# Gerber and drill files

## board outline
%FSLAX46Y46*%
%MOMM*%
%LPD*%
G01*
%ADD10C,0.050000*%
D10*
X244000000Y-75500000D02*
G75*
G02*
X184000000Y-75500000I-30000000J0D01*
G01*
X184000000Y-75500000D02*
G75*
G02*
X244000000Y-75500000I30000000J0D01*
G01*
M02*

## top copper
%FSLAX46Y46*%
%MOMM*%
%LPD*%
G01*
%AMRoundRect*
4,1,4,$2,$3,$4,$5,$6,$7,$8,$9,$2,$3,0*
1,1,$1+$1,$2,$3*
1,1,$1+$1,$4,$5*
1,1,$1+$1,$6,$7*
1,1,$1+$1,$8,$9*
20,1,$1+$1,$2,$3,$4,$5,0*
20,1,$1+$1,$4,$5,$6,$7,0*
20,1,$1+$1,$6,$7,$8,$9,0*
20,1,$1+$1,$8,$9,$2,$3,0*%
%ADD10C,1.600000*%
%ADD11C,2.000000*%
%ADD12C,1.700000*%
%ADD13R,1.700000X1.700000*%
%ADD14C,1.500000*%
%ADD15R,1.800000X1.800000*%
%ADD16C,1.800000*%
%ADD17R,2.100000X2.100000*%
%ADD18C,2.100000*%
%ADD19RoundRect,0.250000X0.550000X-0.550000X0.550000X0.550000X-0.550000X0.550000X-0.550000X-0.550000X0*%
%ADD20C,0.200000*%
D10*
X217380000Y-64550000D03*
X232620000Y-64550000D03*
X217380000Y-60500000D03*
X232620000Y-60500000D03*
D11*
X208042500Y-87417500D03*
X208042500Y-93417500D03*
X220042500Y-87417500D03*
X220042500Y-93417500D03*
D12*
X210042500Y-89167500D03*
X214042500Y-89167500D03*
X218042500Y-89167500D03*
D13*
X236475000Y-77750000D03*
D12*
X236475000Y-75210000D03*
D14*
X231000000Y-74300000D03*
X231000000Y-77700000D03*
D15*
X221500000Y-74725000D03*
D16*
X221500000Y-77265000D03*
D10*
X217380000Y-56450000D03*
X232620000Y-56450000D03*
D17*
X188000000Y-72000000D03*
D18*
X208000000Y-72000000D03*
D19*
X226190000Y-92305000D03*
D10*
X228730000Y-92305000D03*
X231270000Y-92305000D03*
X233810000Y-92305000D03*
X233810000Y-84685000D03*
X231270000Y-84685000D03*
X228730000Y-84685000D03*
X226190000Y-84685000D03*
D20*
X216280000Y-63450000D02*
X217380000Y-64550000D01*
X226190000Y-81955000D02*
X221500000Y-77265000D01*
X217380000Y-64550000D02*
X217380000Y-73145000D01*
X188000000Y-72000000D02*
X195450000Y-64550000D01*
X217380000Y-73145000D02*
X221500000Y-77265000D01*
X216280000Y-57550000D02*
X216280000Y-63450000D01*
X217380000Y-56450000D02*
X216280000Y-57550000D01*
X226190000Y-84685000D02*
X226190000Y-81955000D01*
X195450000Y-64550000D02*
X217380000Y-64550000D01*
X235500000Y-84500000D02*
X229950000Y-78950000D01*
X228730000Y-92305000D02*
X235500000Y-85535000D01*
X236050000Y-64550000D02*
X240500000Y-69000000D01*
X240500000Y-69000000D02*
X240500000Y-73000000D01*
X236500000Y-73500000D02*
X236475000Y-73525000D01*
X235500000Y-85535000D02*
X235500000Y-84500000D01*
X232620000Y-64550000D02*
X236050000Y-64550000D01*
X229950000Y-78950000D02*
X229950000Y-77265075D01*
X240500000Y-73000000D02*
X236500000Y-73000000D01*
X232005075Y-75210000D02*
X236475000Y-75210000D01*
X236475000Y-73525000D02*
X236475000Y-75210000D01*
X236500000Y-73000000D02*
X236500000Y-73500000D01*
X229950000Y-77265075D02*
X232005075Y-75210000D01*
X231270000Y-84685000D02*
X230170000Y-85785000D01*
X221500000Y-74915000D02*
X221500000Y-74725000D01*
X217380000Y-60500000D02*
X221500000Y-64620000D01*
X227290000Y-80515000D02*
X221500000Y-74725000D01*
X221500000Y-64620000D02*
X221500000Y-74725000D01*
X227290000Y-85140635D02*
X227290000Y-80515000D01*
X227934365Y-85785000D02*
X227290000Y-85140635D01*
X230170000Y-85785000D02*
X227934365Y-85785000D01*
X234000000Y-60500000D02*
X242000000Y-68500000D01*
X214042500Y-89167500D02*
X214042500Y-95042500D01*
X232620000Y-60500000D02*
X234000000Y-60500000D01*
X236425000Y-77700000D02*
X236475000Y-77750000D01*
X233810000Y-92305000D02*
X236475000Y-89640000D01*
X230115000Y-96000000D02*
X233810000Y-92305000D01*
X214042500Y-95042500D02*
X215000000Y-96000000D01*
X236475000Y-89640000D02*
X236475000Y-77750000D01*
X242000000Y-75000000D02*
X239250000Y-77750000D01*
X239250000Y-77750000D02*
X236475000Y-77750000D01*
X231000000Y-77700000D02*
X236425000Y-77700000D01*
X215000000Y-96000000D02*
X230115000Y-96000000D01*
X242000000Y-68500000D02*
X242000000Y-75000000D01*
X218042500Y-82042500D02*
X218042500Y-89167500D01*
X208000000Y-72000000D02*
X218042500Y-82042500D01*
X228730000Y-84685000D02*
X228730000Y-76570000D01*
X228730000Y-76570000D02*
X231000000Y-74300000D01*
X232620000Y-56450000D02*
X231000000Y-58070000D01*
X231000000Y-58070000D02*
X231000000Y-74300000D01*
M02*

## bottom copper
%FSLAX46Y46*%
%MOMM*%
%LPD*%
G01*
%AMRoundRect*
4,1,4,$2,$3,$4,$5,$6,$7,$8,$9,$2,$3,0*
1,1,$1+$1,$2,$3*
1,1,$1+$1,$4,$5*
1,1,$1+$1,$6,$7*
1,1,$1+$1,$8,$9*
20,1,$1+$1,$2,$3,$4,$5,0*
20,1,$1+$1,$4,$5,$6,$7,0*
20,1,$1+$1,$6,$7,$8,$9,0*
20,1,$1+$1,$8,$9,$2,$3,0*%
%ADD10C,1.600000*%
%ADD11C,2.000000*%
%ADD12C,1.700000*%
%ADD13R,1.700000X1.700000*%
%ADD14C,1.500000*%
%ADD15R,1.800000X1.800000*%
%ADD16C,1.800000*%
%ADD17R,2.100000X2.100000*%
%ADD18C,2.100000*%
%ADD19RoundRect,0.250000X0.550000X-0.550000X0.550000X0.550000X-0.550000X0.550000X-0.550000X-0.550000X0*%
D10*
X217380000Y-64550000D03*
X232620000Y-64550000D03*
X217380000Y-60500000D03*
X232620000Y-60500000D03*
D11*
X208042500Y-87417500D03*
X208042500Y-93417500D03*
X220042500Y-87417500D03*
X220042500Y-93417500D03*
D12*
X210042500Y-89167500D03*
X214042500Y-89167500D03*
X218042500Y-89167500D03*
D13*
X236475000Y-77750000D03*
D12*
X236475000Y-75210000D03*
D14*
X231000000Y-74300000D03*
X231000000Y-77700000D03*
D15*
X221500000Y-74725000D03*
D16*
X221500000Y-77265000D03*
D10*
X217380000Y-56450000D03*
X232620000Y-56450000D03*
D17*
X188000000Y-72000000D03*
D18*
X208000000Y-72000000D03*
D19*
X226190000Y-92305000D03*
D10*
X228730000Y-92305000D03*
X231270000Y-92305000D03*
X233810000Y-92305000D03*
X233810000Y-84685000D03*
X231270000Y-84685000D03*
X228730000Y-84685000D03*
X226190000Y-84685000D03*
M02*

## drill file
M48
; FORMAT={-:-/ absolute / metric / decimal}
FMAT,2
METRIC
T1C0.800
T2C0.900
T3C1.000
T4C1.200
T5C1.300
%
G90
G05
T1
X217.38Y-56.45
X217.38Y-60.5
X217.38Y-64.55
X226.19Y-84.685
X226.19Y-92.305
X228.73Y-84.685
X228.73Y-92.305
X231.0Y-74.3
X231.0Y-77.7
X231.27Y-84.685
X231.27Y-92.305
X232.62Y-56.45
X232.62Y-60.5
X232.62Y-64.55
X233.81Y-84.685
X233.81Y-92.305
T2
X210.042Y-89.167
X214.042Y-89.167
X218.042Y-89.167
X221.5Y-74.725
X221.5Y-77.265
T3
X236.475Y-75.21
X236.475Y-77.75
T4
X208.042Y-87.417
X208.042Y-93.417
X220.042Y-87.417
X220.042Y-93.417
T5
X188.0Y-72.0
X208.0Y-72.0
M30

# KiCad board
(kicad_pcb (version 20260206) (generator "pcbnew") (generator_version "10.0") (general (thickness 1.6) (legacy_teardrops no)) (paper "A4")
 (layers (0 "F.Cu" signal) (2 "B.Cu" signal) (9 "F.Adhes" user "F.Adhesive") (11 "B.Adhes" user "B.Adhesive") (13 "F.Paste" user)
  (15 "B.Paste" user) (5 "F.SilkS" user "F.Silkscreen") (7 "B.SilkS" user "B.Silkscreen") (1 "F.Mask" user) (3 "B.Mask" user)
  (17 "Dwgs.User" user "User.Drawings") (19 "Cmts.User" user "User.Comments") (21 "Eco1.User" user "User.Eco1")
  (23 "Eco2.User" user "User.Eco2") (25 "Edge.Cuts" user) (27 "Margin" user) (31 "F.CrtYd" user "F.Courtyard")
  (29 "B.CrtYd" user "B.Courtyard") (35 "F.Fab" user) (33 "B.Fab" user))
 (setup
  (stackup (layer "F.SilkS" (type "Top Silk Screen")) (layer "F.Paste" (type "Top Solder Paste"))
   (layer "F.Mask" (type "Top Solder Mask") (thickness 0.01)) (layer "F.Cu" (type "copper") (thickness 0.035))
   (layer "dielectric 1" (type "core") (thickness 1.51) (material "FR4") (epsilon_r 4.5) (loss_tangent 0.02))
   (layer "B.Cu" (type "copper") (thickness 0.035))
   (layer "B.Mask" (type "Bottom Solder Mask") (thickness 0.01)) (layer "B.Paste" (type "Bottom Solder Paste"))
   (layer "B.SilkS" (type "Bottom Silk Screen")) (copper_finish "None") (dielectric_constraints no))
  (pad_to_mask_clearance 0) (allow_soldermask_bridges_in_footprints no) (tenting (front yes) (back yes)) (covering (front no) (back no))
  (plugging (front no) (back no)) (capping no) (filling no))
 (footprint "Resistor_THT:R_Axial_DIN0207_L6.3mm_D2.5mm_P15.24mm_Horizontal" (layer "F.Cu") (at 217.38 64.55)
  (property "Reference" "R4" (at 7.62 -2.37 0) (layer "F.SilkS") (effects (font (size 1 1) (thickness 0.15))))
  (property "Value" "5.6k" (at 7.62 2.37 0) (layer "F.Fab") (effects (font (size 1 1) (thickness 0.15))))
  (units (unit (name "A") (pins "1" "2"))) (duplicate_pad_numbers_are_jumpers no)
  (pad "1" thru_hole circle (at 0 0) (size 1.6 1.6) (drill 0.8) (layers "*.Cu" "*.Mask") (remove_unused_layers no) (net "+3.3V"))
  (pad "2" thru_hole circle (at 15.24 0) (size 1.6 1.6) (drill 0.8) (layers "*.Cu" "*.Mask") (remove_unused_layers no) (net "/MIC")))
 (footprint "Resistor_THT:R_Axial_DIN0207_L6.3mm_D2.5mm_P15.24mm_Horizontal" (layer "F.Cu") (at 217.38 60.5)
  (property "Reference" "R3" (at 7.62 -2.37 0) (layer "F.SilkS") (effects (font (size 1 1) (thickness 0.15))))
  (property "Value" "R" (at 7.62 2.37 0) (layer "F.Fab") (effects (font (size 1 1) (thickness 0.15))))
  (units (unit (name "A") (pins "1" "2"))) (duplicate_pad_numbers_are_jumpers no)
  (pad "1" thru_hole circle (at 0 0) (size 1.6 1.6) (drill 0.8) (layers "*.Cu" "*.Mask") (remove_unused_layers no) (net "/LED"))
  (pad "2" thru_hole circle (at 15.24 0) (size 1.6 1.6) (drill 0.8) (layers "*.Cu" "*.Mask") (remove_unused_layers no) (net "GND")))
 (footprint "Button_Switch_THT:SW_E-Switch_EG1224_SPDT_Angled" (layer "F.Cu") (at 210.0425 89.1675)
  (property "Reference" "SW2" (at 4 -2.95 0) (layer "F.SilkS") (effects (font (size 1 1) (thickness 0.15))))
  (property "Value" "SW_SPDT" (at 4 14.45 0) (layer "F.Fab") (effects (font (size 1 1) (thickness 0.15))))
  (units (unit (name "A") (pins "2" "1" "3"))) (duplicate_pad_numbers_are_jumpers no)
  (pad "" thru_hole circle (at -2 -1.75) (size 2 2) (drill 1.2) (layers "*.Cu" "*.Mask") (remove_unused_layers no))
  (pad "" thru_hole circle (at -2 4.25) (size 2 2) (drill 1.2) (layers "*.Cu" "*.Mask") (remove_unused_layers no))
  (pad "" thru_hole circle (at 10 -1.75) (size 2 2) (drill 1.2) (layers "*.Cu" "*.Mask") (remove_unused_layers no))
  (pad "" thru_hole circle (at 10 4.25) (size 2 2) (drill 1.2) (layers "*.Cu" "*.Mask") (remove_unused_layers no))
  (pad "1" thru_hole circle (at 0 0) (size 1.7 1.7) (drill 0.9) (layers "*.Cu" "*.Mask") (remove_unused_layers no)
   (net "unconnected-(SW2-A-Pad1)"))
  (pad "2" thru_hole circle (at 4 0) (size 1.7 1.7) (drill 0.9) (layers "*.Cu" "*.Mask") (remove_unused_layers no) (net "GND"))
  (pad "3" thru_hole circle (at 8 0) (size 1.7 1.7) (drill 0.9) (layers "*.Cu" "*.Mask") (remove_unused_layers no) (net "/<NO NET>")))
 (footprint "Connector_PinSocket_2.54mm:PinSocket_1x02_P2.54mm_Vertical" (layer "F.Cu") (at 236.475 77.75 180)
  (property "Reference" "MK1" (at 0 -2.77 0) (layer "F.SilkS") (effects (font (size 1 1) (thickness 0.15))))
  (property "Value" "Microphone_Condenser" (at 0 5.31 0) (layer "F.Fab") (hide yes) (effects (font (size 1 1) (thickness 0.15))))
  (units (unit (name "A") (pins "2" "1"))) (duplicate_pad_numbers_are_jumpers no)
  (pad "1" thru_hole rect (at 0 0 180) (size 1.7 1.7) (drill 1) (layers "*.Cu" "*.Mask") (remove_unused_layers no) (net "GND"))
  (pad "2" thru_hole circle (at 0 2.54 180) (size 1.7 1.7) (drill 1) (layers "*.Cu" "*.Mask") (remove_unused_layers no) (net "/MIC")))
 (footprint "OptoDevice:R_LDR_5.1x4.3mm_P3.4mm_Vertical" (layer "F.Cu") (at 231 74.3 -90)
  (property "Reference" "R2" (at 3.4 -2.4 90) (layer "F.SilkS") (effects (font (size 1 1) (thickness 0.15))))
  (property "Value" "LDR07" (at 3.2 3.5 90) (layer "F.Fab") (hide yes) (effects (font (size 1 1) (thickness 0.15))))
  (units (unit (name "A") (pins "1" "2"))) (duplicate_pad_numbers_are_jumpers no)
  (pad "1" thru_hole circle (at 0 0 270) (size 1.5 1.5) (drill 0.8) (layers "*.Cu" "*.Mask") (remove_unused_layers no) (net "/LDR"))
  (pad "2" thru_hole circle (at 3.4 0 270) (size 1.5 1.5) (drill 0.8) (layers "*.Cu" "*.Mask") (remove_unused_layers no) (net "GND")))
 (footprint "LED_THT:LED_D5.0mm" (layer "F.Cu") (at 221.5 74.725 -90)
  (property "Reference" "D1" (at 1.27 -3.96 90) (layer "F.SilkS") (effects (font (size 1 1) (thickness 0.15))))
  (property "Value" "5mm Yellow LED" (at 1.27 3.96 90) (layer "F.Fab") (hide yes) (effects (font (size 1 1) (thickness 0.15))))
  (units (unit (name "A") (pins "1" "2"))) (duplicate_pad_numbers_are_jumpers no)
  (pad "1" thru_hole rect (at 0 0 270) (size 1.8 1.8) (drill 0.9) (layers "*.Cu" "*.Mask") (remove_unused_layers no) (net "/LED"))
  (pad "2" thru_hole circle (at 2.54 0 270) (size 1.8 1.8) (drill 0.9) (layers "*.Cu" "*.Mask") (remove_unused_layers no) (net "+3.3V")))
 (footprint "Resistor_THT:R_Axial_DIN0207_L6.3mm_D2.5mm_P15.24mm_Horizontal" (layer "F.Cu") (at 217.38 56.45)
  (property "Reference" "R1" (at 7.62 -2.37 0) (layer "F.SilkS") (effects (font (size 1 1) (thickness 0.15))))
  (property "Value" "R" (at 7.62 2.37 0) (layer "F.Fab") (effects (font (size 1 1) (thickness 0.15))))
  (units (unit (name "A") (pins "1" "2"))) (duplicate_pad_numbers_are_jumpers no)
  (pad "1" thru_hole circle (at 0 0) (size 1.6 1.6) (drill 0.8) (layers "*.Cu" "*.Mask") (remove_unused_layers no) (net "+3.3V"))
  (pad "2" thru_hole circle (at 15.24 0) (size 1.6 1.6) (drill 0.8) (layers "*.Cu" "*.Mask") (remove_unused_layers no) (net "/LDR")))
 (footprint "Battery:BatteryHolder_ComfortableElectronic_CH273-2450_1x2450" (layer "F.Cu") (at 188 72)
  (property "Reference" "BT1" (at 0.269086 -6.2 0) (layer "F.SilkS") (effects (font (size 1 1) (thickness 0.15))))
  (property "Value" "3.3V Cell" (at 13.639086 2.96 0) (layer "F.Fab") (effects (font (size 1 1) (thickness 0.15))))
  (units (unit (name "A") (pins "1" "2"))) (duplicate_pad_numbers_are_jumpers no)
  (pad "1" thru_hole rect (at 0 0 270) (size 2.1 2.1) (drill 1.3) (layers "*.Cu" "*.Mask") (remove_unused_layers no) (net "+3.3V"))
  (pad "2" thru_hole circle (at 20 0 270) (size 2.1 2.1) (drill 1.3) (layers "*.Cu" "*.Mask") (remove_unused_layers no) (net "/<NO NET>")))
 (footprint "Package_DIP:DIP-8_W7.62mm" (layer "F.Cu") (at 226.19 92.305 90)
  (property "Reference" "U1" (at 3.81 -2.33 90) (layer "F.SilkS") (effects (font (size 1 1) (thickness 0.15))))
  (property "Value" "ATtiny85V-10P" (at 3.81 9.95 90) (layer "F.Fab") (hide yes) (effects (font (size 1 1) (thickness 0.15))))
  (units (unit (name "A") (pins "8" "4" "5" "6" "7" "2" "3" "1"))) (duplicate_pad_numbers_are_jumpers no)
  (pad "1" thru_hole roundrect (at 0 0 90) (size 1.6 1.6) (drill 0.8) (layers "*.Cu" "*.Mask") (remove_unused_layers no)
   (roundrect_rratio 0.15625) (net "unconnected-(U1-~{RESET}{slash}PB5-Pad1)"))
  (pad "2" thru_hole circle (at 0 2.54 90) (size 1.6 1.6) (drill 0.8) (layers "*.Cu" "*.Mask") (remove_unused_layers no) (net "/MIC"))
  (pad "3" thru_hole circle (at 0 5.08 90) (size 1.6 1.6) (drill 0.8) (layers "*.Cu" "*.Mask") (remove_unused_layers no)
   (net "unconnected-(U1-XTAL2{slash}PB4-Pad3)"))
  (pad "4" thru_hole circle (at 0 7.62 90) (size 1.6 1.6) (drill 0.8) (layers "*.Cu" "*.Mask") (remove_unused_layers no) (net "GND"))
  (pad "5" thru_hole circle (at 7.62 7.62 90) (size 1.6 1.6) (drill 0.8) (layers "*.Cu" "*.Mask") (remove_unused_layers no)
   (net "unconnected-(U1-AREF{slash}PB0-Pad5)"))
  (pad "6" thru_hole circle (at 7.62 5.08 90) (size 1.6 1.6) (drill 0.8) (layers "*.Cu" "*.Mask") (remove_unused_layers no) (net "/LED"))
  (pad "7" thru_hole circle (at 7.62 2.54 90) (size 1.6 1.6) (drill 0.8) (layers "*.Cu" "*.Mask") (remove_unused_layers no) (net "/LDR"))
  (pad "8" thru_hole circle (at 7.62 0 90) (size 1.6 1.6) (drill 0.8) (layers "*.Cu" "*.Mask") (remove_unused_layers no) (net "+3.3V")))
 (gr_circle (center 214 75.5) (end 244 75.5) (stroke (width 0.05) (type solid)) (fill no) (locked yes) (layer "Edge.Cuts"))
 (segment (start 216.28 63.45) (end 217.38 64.55) (width 0.2) (layer "F.Cu") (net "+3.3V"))
 (segment (start 226.19 81.955) (end 221.5 77.265) (width 0.2) (layer "F.Cu") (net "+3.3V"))
 (segment (start 217.38 64.55) (end 217.38 73.145) (width 0.2) (layer "F.Cu") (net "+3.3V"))
 (segment (start 188 72) (end 195.45 64.55) (width 0.2) (layer "F.Cu") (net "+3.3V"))
 (segment (start 217.38 73.145) (end 221.5 77.265) (width 0.2) (layer "F.Cu") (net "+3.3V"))
 (segment (start 216.28 57.55) (end 216.28 63.45) (width 0.2) (layer "F.Cu") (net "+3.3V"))
 (segment (start 217.38 56.45) (end 216.28 57.55) (width 0.2) (layer "F.Cu") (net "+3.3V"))
 (segment (start 226.19 84.685) (end 226.19 81.955) (width 0.2) (layer "F.Cu") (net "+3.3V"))
 (segment (start 195.45 64.55) (end 217.38 64.55) (width 0.2) (layer "F.Cu") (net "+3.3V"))
 (segment (start 235.5 84.5) (end 229.95 78.95) (width 0.2) (layer "F.Cu") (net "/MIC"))
 (segment (start 228.73 92.305) (end 235.5 85.535) (width 0.2) (layer "F.Cu") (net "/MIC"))
 (segment (start 236.05 64.55) (end 240.5 69) (width 0.2) (layer "F.Cu") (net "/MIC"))
 (segment (start 240.5 69) (end 240.5 73) (width 0.2) (layer "F.Cu") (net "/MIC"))
 (segment (start 236.5 73.5) (end 236.475 73.525) (width 0.2) (layer "F.Cu") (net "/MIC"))
 (segment (start 235.5 85.535) (end 235.5 84.5) (width 0.2) (layer "F.Cu") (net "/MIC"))
 (segment (start 232.62 64.55) (end 236.05 64.55) (width 0.2) (layer "F.Cu") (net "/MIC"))
 (segment (start 229.95 78.95) (end 229.95 77.265075) (width 0.2) (layer "F.Cu") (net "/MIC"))
 (segment (start 240.5 73) (end 236.5 73) (width 0.2) (layer "F.Cu") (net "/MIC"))
 (segment (start 232.005075 75.21) (end 236.475 75.21) (width 0.2) (layer "F.Cu") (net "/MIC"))
 (segment (start 236.475 73.525) (end 236.475 75.21) (width 0.2) (layer "F.Cu") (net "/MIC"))
 (segment (start 236.5 73) (end 236.5 73.5) (width 0.2) (layer "F.Cu") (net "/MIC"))
 (segment (start 229.95 77.265075) (end 232.005075 75.21) (width 0.2) (layer "F.Cu") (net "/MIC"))
 (segment (start 231.27 84.685) (end 230.17 85.785) (width 0.2) (layer "F.Cu") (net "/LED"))
 (segment (start 221.5 74.915) (end 221.5 74.725) (width 0.2) (layer "F.Cu") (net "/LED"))
 (segment (start 217.38 60.5) (end 221.5 64.62) (width 0.2) (layer "F.Cu") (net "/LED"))
 (segment (start 227.29 80.515) (end 221.5 74.725) (width 0.2) (layer "F.Cu") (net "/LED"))
 (segment (start 221.5 64.62) (end 221.5 74.725) (width 0.2) (layer "F.Cu") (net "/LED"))
 (segment (start 227.29 85.140635) (end 227.29 80.515) (width 0.2) (layer "F.Cu") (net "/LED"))
 (segment (start 227.934365 85.785) (end 227.29 85.140635) (width 0.2) (layer "F.Cu") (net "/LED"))
 (segment (start 230.17 85.785) (end 227.934365 85.785) (width 0.2) (layer "F.Cu") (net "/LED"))
 (segment (start 234 60.5) (end 242 68.5) (width 0.2) (layer "F.Cu") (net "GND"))
 (segment (start 214.0425 89.1675) (end 214.0425 95.0425) (width 0.2) (layer "F.Cu") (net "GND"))
 (segment (start 232.62 60.5) (end 234 60.5) (width 0.2) (layer "F.Cu") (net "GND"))
 (segment (start 236.425 77.7) (end 236.475 77.75) (width 0.2) (layer "F.Cu") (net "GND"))
 (segment (start 233.81 92.305) (end 236.475 89.64) (width 0.2) (layer "F.Cu") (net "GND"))
 (segment (start 230.115 96) (end 233.81 92.305) (width 0.2) (layer "F.Cu") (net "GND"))
 (segment (start 214.0425 95.0425) (end 215 96) (width 0.2) (layer "F.Cu") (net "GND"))
 (segment (start 236.475 89.64) (end 236.475 77.75) (width 0.2) (layer "F.Cu") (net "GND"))
 (segment (start 242 75) (end 239.25 77.75) (width 0.2) (layer "F.Cu") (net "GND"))
 (segment (start 239.25 77.75) (end 236.475 77.75) (width 0.2) (layer "F.Cu") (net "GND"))
 (segment (start 231 77.7) (end 236.425 77.7) (width 0.2) (layer "F.Cu") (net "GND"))
 (segment (start 215 96) (end 230.115 96) (width 0.2) (layer "F.Cu") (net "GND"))
 (segment (start 242 68.5) (end 242 75) (width 0.2) (layer "F.Cu") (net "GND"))
 (segment (start 218.0425 82.0425) (end 218.0425 89.1675) (width 0.2) (layer "F.Cu") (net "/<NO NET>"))
 (segment (start 208 72) (end 218.0425 82.0425) (width 0.2) (layer "F.Cu") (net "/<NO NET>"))
 (segment (start 228.73 84.685) (end 228.73 76.57) (width 0.2) (layer "F.Cu") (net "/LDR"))
 (segment (start 228.73 76.57) (end 231 74.3) (width 0.2) (layer "F.Cu") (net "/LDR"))
 (segment (start 232.62 56.45) (end 231 58.07) (width 0.2) (layer "F.Cu") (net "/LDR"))
 (segment (start 231 58.07) (end 231 74.3) (width 0.2) (layer "F.Cu") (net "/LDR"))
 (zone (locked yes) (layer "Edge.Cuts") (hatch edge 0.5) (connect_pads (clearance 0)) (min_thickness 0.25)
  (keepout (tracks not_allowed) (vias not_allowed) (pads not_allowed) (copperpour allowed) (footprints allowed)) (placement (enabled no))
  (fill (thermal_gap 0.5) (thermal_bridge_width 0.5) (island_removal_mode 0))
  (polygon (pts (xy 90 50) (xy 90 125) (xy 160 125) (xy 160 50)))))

